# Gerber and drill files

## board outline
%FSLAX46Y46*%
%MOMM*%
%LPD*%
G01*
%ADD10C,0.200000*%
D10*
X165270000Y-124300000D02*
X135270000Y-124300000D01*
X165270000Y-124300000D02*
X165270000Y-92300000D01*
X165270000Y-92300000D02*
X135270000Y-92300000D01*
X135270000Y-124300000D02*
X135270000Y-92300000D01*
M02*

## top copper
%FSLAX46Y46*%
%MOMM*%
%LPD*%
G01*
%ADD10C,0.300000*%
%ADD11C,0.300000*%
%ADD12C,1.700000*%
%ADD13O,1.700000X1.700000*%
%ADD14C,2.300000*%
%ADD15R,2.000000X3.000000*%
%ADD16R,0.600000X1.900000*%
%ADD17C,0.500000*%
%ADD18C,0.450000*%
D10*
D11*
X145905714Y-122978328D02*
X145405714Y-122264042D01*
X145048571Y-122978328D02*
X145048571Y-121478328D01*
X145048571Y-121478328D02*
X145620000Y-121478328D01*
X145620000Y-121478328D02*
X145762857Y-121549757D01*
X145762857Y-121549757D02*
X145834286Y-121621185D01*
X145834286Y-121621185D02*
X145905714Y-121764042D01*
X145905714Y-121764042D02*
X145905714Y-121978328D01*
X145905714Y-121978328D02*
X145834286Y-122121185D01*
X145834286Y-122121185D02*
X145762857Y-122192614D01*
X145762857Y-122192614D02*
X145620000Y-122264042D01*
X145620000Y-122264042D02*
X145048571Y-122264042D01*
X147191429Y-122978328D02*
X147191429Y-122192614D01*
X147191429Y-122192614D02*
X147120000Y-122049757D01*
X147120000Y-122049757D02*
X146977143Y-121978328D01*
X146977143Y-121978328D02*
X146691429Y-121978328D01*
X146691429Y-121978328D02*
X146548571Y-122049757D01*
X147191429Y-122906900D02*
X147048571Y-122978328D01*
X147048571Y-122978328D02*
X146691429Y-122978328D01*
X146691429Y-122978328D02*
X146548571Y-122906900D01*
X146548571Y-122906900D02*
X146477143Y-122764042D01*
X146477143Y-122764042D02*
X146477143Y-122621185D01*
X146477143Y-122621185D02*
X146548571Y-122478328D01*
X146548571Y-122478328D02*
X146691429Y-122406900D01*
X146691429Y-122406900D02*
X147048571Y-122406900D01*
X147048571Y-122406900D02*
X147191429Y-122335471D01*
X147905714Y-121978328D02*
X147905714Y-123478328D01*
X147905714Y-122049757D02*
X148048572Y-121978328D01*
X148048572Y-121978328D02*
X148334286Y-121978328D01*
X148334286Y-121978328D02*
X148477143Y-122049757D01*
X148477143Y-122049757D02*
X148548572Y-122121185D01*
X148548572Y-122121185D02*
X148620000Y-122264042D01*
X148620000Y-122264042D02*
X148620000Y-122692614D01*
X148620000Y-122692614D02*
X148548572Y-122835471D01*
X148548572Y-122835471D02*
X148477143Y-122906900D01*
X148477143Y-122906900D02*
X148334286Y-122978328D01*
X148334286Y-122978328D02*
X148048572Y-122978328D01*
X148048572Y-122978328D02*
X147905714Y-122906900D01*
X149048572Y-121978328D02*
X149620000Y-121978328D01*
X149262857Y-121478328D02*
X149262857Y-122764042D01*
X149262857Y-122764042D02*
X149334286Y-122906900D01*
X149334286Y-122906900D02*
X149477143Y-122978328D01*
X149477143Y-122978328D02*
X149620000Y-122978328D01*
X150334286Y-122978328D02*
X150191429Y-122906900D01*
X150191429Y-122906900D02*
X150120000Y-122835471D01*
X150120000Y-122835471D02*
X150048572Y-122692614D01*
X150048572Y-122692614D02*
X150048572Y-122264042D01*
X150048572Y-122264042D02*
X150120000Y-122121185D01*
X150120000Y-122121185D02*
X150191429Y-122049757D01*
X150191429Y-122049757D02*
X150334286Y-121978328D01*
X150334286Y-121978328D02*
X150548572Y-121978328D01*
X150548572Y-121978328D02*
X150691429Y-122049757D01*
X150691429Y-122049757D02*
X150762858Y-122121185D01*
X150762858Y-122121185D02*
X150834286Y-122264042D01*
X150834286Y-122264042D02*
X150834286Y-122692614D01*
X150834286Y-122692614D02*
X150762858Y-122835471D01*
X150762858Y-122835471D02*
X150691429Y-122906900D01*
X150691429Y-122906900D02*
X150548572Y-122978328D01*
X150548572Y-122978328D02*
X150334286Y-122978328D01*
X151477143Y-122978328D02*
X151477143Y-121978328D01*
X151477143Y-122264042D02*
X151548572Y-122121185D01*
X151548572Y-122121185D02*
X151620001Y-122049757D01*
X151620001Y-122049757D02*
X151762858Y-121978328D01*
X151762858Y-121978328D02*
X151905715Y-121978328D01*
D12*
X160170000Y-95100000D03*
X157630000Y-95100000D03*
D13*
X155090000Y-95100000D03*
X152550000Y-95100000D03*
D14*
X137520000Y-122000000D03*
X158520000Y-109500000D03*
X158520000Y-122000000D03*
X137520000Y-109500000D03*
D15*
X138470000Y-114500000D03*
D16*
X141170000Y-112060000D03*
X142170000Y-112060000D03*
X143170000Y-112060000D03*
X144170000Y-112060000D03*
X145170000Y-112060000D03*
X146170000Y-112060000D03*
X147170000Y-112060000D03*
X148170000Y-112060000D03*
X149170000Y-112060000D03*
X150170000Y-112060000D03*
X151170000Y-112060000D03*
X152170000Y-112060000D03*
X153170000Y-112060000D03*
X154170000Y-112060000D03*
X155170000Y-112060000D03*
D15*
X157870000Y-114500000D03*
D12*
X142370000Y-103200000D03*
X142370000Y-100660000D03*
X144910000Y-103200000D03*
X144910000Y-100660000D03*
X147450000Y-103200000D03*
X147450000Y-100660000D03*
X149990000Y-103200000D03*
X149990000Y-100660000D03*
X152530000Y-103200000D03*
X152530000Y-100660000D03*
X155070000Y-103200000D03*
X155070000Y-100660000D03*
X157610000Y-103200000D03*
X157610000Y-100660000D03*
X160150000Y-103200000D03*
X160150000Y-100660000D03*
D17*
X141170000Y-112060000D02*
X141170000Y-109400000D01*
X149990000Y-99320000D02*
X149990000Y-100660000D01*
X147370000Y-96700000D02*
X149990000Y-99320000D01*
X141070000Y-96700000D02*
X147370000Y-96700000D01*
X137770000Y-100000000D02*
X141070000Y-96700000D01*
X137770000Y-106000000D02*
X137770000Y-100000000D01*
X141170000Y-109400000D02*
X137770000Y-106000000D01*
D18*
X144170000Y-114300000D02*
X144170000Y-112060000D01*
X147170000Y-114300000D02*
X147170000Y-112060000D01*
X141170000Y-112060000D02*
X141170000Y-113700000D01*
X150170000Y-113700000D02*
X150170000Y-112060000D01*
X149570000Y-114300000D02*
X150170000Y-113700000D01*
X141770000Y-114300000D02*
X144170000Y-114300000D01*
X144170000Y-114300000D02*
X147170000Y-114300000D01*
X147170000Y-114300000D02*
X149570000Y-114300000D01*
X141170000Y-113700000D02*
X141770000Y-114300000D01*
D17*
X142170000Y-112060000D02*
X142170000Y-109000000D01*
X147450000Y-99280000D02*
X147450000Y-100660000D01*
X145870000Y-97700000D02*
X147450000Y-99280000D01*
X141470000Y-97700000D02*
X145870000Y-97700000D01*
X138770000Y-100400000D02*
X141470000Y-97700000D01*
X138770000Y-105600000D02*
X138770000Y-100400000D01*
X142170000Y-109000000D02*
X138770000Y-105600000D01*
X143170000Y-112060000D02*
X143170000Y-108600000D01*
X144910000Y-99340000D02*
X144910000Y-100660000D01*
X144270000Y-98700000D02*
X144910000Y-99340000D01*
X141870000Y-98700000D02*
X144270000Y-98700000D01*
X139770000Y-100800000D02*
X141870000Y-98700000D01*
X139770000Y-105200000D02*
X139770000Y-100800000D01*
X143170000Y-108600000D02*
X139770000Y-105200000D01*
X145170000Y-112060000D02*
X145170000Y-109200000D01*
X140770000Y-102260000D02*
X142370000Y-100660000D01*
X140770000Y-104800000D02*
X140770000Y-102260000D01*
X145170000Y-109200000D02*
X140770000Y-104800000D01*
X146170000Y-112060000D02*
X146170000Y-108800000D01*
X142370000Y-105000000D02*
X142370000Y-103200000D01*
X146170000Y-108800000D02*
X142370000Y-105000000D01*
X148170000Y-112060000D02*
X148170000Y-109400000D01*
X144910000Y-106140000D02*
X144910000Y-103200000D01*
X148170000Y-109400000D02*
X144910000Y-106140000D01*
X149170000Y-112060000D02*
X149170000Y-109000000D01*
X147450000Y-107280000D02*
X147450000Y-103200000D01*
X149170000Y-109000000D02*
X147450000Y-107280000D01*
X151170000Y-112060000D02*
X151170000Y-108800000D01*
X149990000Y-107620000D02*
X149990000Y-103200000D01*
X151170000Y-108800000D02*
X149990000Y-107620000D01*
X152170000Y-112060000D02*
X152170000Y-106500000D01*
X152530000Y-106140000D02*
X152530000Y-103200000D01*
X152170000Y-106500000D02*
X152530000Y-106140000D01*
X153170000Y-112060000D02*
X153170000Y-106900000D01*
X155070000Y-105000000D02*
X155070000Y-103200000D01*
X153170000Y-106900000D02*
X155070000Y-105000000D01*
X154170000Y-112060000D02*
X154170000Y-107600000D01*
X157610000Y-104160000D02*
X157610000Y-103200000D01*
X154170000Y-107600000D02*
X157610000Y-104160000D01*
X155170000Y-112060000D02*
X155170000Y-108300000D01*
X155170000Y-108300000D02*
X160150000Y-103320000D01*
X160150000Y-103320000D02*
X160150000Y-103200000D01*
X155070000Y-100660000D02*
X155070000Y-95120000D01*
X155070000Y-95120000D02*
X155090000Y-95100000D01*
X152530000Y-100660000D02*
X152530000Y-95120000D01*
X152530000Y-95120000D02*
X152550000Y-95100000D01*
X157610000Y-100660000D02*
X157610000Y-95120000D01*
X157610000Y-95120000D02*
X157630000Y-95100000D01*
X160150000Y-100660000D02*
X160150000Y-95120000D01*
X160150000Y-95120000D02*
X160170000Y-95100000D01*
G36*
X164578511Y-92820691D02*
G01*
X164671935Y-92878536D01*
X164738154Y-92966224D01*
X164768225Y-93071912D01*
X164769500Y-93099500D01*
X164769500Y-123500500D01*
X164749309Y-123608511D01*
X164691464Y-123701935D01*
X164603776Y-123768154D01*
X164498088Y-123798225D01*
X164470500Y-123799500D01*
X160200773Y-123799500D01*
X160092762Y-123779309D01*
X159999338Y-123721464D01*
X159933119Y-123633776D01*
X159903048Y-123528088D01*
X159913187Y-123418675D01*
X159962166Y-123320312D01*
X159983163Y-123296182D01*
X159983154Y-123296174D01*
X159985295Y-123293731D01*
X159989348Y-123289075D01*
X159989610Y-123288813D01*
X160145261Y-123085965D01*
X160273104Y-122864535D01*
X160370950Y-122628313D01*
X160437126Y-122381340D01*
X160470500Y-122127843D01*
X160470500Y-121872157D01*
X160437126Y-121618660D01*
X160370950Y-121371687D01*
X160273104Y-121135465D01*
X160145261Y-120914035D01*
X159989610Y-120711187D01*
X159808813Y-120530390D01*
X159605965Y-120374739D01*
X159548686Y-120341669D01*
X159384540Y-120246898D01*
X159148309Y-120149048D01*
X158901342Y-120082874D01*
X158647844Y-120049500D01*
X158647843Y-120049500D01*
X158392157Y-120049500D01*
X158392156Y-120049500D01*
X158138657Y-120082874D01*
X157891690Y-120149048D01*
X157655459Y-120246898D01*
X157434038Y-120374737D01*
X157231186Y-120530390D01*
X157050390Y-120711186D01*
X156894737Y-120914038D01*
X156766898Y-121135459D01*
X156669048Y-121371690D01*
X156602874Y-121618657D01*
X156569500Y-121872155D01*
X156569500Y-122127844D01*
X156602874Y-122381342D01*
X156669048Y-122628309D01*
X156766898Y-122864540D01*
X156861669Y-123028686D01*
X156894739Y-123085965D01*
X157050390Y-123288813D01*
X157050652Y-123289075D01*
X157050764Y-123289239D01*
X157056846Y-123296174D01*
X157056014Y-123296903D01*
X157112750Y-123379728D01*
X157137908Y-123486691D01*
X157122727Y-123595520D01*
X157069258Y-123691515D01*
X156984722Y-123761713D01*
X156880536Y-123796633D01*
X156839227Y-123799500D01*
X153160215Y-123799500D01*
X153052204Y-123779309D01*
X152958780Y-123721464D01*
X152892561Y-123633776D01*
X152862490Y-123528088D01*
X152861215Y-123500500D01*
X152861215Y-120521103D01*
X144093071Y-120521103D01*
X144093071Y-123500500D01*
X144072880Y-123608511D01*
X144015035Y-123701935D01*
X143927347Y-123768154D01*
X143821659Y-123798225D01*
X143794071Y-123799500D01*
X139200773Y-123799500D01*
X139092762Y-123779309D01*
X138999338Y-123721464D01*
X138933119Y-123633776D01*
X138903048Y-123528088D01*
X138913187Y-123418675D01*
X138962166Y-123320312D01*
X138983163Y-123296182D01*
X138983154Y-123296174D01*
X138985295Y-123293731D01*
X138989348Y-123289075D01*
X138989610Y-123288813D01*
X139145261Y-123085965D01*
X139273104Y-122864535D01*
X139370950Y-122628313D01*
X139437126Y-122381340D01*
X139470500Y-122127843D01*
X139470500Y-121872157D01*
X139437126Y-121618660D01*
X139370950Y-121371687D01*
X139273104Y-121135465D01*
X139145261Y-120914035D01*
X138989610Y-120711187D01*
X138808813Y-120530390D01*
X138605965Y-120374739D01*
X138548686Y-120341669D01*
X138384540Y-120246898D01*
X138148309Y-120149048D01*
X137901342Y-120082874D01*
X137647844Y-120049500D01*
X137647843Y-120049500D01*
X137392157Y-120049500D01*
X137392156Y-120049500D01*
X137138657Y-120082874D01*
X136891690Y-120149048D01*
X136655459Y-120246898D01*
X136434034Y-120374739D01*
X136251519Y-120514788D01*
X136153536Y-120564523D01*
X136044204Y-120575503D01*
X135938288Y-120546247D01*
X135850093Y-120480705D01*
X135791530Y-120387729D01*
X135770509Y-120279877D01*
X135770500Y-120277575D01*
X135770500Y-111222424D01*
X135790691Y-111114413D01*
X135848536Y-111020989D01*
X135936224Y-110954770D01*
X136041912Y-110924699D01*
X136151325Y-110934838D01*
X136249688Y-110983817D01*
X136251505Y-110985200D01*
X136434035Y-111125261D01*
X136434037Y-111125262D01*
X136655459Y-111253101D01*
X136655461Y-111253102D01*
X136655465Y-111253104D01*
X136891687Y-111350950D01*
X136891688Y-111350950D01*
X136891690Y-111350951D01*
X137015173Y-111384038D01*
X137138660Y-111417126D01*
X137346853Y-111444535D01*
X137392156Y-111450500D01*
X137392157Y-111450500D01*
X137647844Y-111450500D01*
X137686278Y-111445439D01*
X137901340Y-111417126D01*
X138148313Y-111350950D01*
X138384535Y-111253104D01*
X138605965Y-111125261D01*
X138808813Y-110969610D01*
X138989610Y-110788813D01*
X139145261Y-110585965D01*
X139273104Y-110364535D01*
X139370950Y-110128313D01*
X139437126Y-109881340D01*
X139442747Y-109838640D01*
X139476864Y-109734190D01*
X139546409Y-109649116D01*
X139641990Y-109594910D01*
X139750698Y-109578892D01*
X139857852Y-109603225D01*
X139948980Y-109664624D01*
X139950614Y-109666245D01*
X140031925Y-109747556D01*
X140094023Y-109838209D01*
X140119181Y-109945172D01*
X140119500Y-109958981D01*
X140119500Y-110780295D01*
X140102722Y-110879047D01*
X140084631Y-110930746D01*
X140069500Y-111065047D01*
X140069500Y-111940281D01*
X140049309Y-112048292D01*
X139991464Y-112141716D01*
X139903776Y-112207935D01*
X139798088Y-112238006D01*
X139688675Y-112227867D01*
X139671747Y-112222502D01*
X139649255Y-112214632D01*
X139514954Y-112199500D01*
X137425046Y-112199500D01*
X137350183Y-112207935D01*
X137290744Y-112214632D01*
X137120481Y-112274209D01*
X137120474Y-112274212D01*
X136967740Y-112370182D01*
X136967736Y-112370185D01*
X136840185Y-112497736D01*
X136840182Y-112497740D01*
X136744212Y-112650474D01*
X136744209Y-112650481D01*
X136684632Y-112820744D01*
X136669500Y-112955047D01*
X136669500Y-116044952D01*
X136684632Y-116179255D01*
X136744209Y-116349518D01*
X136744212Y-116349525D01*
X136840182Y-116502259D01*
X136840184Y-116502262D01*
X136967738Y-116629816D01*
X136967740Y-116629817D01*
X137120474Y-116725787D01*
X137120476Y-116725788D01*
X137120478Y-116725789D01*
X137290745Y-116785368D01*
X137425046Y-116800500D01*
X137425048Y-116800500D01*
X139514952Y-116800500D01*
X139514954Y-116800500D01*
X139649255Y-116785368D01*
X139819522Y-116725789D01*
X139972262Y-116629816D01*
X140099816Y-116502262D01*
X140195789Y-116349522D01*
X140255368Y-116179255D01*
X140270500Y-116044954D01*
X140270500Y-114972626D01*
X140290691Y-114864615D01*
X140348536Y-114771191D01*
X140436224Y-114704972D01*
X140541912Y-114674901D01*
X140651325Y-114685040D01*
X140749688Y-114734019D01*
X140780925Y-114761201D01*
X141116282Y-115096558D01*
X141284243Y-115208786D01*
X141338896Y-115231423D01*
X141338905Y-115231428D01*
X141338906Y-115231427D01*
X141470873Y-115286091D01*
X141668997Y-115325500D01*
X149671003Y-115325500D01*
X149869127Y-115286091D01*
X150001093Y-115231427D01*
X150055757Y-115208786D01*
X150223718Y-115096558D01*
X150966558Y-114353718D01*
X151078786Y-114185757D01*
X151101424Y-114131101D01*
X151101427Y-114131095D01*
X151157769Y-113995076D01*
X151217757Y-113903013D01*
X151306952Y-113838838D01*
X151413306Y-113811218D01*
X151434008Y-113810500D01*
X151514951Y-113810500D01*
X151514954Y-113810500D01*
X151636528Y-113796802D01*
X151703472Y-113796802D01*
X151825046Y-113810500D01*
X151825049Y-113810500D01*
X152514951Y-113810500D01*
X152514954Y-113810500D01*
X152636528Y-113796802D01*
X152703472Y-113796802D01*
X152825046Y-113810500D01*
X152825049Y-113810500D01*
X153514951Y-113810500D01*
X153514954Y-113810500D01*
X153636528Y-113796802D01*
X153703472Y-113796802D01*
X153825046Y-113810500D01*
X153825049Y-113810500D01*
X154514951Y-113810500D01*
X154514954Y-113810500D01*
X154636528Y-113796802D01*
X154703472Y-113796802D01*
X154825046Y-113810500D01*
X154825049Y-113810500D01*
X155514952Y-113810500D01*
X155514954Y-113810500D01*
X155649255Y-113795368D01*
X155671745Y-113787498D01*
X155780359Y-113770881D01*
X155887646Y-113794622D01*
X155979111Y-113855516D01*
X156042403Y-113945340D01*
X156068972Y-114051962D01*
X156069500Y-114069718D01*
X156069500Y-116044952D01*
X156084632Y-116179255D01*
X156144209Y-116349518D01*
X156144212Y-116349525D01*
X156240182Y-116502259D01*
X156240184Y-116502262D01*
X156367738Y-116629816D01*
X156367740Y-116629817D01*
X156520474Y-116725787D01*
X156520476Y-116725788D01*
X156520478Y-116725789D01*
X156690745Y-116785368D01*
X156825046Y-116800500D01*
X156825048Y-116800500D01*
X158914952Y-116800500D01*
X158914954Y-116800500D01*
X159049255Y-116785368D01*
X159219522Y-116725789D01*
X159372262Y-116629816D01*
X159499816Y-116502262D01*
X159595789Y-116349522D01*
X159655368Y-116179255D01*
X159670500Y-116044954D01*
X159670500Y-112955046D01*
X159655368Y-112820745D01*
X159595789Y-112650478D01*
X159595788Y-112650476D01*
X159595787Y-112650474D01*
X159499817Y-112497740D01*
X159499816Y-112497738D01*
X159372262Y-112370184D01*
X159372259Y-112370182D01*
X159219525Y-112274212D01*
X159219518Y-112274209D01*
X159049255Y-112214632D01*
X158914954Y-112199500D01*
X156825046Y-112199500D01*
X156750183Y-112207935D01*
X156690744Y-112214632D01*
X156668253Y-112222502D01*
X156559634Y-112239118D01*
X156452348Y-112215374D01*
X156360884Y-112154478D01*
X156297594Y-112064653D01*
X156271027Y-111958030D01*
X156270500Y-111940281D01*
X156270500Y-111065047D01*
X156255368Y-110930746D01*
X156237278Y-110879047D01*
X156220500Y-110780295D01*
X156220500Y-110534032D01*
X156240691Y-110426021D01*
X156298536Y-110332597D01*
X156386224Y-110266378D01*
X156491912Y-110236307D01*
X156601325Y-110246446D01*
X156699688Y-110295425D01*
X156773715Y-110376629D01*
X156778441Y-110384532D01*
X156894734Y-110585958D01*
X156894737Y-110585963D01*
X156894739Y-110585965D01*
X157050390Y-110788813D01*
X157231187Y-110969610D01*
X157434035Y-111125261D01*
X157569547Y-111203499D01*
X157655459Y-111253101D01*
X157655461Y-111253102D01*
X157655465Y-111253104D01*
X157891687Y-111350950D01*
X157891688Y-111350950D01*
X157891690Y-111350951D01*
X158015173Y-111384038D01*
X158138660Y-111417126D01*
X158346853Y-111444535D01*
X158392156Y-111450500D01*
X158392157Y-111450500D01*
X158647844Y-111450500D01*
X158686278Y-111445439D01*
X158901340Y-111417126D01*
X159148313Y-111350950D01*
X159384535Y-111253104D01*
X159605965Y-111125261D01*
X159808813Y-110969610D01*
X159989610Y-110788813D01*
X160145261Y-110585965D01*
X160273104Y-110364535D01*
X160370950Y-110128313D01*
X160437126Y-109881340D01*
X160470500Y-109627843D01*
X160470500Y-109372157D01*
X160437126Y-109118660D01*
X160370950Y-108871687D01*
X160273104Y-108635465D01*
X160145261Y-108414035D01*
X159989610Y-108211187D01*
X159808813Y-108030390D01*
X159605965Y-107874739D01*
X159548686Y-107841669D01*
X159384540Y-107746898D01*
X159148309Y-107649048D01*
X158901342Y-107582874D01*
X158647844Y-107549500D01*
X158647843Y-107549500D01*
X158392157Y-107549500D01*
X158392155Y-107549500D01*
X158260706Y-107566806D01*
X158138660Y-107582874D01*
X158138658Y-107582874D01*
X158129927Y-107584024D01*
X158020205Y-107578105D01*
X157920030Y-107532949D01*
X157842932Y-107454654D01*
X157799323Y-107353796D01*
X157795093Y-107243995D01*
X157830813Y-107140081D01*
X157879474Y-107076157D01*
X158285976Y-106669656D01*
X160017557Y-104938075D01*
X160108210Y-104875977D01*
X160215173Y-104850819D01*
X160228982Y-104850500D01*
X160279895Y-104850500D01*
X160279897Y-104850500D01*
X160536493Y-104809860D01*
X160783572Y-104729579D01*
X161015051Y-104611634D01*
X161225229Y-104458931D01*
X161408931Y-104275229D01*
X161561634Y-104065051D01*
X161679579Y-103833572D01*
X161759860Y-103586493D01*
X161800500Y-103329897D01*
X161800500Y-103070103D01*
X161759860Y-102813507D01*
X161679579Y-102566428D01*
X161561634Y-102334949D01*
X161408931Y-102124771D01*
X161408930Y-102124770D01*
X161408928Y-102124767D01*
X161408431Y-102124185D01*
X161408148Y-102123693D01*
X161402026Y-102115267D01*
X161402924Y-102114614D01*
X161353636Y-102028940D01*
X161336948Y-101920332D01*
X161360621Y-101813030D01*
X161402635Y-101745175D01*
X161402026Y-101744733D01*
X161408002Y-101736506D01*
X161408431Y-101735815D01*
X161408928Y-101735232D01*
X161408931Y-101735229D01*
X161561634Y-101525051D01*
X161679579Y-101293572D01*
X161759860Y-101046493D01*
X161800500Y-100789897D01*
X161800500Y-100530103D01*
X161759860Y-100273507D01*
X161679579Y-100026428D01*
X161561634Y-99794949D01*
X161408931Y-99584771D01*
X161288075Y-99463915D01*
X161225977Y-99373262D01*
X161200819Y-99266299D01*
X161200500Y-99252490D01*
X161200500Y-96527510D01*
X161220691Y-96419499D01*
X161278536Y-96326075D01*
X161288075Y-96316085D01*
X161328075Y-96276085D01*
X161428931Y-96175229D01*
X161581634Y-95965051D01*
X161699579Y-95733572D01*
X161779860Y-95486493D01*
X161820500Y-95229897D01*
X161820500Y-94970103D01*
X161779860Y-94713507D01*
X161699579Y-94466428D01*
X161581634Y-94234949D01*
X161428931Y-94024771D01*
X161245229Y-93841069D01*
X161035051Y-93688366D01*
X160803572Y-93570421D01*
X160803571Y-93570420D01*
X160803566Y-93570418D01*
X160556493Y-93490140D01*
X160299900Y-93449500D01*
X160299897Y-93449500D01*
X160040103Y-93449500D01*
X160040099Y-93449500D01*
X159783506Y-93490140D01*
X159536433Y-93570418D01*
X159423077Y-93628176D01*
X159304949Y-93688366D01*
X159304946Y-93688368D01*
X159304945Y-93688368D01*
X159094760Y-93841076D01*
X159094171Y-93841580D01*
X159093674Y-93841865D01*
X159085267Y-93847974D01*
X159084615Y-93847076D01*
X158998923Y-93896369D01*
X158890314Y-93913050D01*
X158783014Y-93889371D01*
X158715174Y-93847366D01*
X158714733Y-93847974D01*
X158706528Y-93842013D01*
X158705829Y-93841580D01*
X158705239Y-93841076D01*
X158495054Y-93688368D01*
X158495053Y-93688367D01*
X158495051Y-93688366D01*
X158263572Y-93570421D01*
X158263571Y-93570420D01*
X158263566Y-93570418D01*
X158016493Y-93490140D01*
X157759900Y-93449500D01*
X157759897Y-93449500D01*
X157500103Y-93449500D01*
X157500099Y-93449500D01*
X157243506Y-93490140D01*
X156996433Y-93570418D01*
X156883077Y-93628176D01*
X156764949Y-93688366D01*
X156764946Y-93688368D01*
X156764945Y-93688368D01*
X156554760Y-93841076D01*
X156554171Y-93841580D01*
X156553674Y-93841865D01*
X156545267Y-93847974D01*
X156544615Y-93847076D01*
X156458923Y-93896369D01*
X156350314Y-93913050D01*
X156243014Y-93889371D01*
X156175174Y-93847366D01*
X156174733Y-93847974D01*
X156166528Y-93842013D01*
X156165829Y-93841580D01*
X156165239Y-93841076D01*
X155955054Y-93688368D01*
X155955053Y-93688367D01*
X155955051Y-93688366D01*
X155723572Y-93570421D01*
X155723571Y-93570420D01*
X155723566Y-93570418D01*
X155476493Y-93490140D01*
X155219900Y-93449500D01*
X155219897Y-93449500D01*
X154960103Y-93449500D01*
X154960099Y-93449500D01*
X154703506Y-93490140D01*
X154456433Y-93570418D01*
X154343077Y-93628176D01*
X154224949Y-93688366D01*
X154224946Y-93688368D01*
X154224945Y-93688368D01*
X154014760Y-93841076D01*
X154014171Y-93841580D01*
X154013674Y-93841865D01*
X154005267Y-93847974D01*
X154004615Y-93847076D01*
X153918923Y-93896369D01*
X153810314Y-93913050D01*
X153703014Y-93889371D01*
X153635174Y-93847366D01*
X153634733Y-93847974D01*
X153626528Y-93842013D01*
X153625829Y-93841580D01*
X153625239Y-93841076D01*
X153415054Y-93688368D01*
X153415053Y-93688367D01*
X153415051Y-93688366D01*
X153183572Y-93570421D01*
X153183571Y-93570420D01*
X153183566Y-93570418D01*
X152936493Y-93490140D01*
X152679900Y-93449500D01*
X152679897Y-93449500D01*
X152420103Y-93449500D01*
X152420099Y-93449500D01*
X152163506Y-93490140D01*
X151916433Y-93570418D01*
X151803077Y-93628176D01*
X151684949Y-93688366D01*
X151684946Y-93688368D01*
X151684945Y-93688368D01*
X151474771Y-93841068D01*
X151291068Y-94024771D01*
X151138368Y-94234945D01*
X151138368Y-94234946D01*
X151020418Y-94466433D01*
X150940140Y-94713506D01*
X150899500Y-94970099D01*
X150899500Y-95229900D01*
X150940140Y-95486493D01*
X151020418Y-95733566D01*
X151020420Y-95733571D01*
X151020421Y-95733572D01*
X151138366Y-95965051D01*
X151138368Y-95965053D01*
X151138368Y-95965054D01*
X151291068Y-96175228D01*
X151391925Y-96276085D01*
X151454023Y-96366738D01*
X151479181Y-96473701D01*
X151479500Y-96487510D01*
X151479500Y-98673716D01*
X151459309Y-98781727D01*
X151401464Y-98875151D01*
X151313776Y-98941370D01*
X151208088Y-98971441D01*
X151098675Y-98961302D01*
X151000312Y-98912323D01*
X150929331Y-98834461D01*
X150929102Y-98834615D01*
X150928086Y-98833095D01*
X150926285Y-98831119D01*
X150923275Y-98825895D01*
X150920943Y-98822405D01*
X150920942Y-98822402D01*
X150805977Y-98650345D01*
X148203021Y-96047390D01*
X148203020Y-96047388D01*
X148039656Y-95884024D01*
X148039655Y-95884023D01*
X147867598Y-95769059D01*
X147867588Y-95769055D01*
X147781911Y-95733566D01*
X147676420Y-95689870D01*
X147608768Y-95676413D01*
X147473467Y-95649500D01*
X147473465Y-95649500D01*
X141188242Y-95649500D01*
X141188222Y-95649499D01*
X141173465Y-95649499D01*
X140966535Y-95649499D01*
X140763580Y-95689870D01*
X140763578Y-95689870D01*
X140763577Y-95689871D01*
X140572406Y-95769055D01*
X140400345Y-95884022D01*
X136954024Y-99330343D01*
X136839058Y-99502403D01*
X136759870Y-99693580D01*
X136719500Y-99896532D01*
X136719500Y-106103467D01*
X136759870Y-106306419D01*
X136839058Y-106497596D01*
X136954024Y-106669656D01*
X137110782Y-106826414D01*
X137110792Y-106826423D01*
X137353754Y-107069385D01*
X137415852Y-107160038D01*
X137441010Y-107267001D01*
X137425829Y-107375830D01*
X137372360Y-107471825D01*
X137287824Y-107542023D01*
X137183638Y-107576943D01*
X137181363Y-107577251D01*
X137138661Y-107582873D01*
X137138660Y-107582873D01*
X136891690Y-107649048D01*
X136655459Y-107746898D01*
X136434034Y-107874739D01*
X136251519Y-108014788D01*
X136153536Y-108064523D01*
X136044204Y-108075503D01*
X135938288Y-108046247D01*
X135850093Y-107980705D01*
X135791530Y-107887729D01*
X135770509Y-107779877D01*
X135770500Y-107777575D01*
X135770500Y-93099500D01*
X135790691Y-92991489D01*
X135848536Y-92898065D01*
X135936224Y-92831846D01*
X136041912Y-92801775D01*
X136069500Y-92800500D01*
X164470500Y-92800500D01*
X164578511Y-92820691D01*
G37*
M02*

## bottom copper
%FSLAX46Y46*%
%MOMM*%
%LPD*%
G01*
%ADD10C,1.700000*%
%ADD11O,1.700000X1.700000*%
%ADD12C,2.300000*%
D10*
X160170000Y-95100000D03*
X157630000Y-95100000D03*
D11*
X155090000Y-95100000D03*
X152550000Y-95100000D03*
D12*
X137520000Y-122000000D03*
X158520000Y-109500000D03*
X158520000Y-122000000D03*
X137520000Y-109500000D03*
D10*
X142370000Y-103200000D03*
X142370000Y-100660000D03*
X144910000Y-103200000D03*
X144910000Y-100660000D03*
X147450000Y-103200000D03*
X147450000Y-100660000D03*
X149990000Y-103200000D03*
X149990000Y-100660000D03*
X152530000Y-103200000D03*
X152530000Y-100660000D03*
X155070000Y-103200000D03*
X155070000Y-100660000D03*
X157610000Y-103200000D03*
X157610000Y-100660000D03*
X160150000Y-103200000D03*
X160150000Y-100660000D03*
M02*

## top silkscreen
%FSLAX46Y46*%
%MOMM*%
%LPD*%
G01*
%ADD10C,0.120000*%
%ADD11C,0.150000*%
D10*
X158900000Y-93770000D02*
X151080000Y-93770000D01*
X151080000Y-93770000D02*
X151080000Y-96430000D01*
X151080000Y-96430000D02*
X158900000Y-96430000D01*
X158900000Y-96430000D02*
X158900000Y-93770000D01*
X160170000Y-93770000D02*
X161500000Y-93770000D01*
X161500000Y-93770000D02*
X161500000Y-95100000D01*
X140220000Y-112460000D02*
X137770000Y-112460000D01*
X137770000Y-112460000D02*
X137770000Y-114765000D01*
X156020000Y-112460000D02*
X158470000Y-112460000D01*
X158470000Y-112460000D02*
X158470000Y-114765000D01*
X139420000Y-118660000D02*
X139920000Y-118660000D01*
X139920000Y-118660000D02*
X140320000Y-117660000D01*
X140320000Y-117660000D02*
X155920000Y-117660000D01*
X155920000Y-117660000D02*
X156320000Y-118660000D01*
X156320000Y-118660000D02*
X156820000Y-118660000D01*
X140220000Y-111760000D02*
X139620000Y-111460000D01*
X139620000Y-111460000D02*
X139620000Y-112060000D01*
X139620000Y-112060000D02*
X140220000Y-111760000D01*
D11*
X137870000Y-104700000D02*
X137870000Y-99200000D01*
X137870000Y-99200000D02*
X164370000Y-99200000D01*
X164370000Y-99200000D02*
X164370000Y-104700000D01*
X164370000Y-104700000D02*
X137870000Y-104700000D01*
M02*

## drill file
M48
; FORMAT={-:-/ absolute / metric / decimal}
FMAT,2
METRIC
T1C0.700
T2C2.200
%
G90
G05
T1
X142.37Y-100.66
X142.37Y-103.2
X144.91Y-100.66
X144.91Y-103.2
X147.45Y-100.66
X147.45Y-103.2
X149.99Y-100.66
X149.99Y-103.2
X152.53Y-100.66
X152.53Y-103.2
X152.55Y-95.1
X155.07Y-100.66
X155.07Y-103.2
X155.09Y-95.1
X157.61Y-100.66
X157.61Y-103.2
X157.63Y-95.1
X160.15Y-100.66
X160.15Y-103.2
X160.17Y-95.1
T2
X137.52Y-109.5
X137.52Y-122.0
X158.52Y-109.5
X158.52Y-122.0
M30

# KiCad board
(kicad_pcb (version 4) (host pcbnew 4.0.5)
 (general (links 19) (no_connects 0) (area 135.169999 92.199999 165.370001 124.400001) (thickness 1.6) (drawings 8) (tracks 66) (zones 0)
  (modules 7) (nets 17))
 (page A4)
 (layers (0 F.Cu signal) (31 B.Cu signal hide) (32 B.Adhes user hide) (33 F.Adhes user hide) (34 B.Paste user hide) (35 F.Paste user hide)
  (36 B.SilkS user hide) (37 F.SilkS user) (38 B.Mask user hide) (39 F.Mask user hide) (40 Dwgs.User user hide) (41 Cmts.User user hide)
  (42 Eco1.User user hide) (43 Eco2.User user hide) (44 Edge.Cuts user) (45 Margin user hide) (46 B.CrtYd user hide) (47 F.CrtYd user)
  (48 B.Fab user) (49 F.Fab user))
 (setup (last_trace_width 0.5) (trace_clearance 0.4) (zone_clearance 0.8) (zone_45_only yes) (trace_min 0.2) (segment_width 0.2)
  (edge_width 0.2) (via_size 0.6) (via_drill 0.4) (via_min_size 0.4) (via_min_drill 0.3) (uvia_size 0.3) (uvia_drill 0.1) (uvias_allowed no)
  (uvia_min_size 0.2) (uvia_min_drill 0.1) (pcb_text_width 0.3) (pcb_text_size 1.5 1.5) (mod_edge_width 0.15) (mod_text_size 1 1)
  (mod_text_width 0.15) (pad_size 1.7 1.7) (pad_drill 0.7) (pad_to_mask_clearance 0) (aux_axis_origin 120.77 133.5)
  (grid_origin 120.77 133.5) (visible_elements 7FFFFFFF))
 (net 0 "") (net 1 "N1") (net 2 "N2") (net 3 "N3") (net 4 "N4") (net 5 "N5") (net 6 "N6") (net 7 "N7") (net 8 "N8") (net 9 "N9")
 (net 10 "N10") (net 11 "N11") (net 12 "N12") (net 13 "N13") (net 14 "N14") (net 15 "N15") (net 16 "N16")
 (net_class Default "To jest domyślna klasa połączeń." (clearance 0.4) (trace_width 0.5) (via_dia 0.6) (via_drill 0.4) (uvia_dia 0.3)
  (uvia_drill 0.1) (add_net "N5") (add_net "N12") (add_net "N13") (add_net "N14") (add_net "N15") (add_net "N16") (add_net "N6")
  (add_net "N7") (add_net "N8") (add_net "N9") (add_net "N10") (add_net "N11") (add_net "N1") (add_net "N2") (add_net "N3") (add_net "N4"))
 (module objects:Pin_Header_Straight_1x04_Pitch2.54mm (layer F.Cu) (at 160.17 95.1 270)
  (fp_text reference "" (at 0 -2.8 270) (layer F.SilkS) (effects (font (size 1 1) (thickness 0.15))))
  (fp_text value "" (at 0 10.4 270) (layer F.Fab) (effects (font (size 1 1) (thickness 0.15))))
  (fp_line (start -1.33 1.27) (end -1.33 9.09) (layer F.SilkS) (width 0.12))
  (fp_line (start -1.33 9.09) (end 1.33 9.09) (layer F.SilkS) (width 0.12))
  (fp_line (start 1.33 9.09) (end 1.33 1.27) (layer F.SilkS) (width 0.12))
  (fp_line (start 1.33 1.27) (end -1.33 1.27) (layer F.SilkS) (width 0.12))
  (fp_line (start -1.33 0) (end -1.33 -1.33) (layer F.SilkS) (width 0.12))
  (fp_line (start -1.33 -1.33) (end 0 -1.33) (layer F.SilkS) (width 0.12))
  (pad 1 thru_hole circle (at 0 0 270) (size 1.7 1.7) (drill 0.7) (layers *.Cu *.Mask) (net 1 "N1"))
  (pad 2 thru_hole circle (at 0 2.54 270) (size 1.7 1.7) (drill 0.7) (layers *.Cu *.Mask) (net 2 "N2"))
  (pad 3 thru_hole oval (at 0 5.08 270) (size 1.7 1.7) (drill 0.7) (layers *.Cu *.Mask) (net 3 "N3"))
  (pad 4 thru_hole oval (at 0 7.62 270) (size 1.7 1.7) (drill 0.7) (layers *.Cu *.Mask) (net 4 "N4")))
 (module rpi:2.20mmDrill (layer F.Cu) (at 137.52 122)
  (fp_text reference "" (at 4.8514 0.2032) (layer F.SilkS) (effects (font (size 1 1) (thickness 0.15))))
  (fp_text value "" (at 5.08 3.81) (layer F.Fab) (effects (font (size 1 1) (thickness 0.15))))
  (pad "" thru_hole circle (at 0 0) (size 2.3 2.3) (drill 2.2) (layers *.Cu *.Mask)))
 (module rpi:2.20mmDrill (layer F.Cu) (at 158.52 109.5)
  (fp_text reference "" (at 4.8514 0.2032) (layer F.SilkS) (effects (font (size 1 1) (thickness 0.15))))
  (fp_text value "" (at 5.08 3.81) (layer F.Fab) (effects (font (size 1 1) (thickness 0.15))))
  (pad "" thru_hole circle (at 0 0) (size 2.3 2.3) (drill 2.2) (layers *.Cu *.Mask)))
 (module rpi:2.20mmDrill (layer F.Cu) (at 158.52 122)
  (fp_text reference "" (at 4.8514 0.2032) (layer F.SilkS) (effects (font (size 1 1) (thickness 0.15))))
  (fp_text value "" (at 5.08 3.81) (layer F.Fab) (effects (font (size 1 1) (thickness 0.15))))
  (pad "" thru_hole circle (at 0 0) (size 2.3 2.3) (drill 2.2) (layers *.Cu *.Mask)))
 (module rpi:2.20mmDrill (layer F.Cu) (at 137.52 109.5)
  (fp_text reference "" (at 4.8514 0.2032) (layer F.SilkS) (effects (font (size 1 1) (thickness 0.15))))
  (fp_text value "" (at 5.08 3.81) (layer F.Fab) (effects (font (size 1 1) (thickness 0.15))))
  (pad "" thru_hole circle (at 0 0) (size 2.3 2.3) (drill 2.2) (layers *.Cu *.Mask)))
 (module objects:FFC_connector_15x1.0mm (layer F.Cu) (at 148.07 114.5)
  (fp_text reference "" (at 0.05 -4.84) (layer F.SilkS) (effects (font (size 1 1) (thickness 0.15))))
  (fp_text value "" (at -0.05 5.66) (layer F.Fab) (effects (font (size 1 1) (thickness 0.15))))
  (fp_line (start -7.85 -2.04) (end -10.3 -2.04) (layer F.SilkS) (width 0.12))
  (fp_line (start -10.3 -2.04) (end -10.3 0.265) (layer F.SilkS) (width 0.12))
  (fp_line (start 7.95 -2.04) (end 10.4 -2.04) (layer F.SilkS) (width 0.12))
  (fp_line (start 10.4 -2.04) (end 10.4 0.265) (layer F.SilkS) (width 0.12))
  (fp_line (start -8.65 4.16) (end -8.15 4.16) (layer F.SilkS) (width 0.12))
  (fp_line (start -8.15 4.16) (end -7.75 3.16) (layer F.SilkS) (width 0.12))
  (fp_line (start -7.75 3.16) (end 7.85 3.16) (layer F.SilkS) (width 0.12))
  (fp_line (start 7.85 3.16) (end 8.25 4.16) (layer F.SilkS) (width 0.12))
  (fp_line (start 8.25 4.16) (end 8.75 4.16) (layer F.SilkS) (width 0.12))
  (fp_line (start -7.85 -2.74) (end -8.45 -3.04) (layer F.SilkS) (width 0.12))
  (fp_line (start -8.45 -3.04) (end -8.45 -2.44) (layer F.SilkS) (width 0.12))
  (fp_line (start -8.45 -2.44) (end -7.85 -2.74) (layer F.SilkS) (width 0.12))
  (pad "" smd rect (at -9.6 0) (size 2 3) (layers F.Cu F.Paste F.Mask))
  (pad 1 smd rect (at -6.9 -2.44) (size 0.6 1.9) (layers F.Cu F.Paste F.Mask) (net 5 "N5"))
  (pad 2 smd rect (at -5.9 -2.44) (size 0.6 1.9) (layers F.Cu F.Paste F.Mask) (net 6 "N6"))
  (pad 3 smd rect (at -4.9 -2.44) (size 0.6 1.9) (layers F.Cu F.Paste F.Mask) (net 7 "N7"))
  (pad 4 smd rect (at -3.9 -2.44) (size 0.6 1.9) (layers F.Cu F.Paste F.Mask) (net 5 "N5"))
  (pad 5 smd rect (at -2.9 -2.44) (size 0.6 1.9) (layers F.Cu F.Paste F.Mask) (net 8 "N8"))
  (pad 6 smd rect (at -1.9 -2.44) (size 0.6 1.9) (layers F.Cu F.Paste F.Mask) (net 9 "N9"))
  (pad 7 smd rect (at -0.9 -2.44) (size 0.6 1.9) (layers F.Cu F.Paste F.Mask) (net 5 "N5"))
  (pad 8 smd rect (at 0.1 -2.44) (size 0.6 1.9) (layers F.Cu F.Paste F.Mask) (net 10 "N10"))
  (pad 9 smd rect (at 1.1 -2.44) (size 0.6 1.9) (layers F.Cu F.Paste F.Mask) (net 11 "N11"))
  (pad 10 smd rect (at 2.1 -2.44) (size 0.6 1.9) (layers F.Cu F.Paste F.Mask) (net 5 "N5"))
  (pad 11 smd rect (at 3.1 -2.44) (size 0.6 1.9) (layers F.Cu F.Paste F.Mask) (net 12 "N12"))
  (pad 12 smd rect (at 4.1 -2.44) (size 0.6 1.9) (layers F.Cu F.Paste F.Mask) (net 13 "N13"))
  (pad 13 smd rect (at 5.1 -2.44) (size 0.6 1.9) (layers F.Cu F.Paste F.Mask) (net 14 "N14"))
  (pad 14 smd rect (at 6.1 -2.44) (size 0.6 1.9) (layers F.Cu F.Paste F.Mask) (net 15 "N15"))
  (pad 15 smd rect (at 7.1 -2.44) (size 0.6 1.9) (layers F.Cu F.Paste F.Mask) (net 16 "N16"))
  (pad "" smd rect (at 9.8 0) (size 2 3) (layers F.Cu F.Paste F.Mask)))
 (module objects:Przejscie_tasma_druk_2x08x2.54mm (layer F.Cu) (at 142.37 103.2)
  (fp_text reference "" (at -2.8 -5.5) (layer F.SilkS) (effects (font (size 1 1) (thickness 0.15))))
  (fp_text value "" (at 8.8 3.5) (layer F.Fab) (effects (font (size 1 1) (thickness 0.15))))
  (fp_line (start -4.5 1.5) (end -4.5 -4) (layer F.SilkS) (width 0.15))
  (fp_line (start -4.5 -4) (end 22 -4) (layer F.SilkS) (width 0.15))
  (fp_line (start 22 -4) (end 22 1.5) (layer F.SilkS) (width 0.15))
  (fp_line (start 22 1.5) (end -4.5 1.5) (layer F.SilkS) (width 0.15))
  (pad 1 thru_hole circle (at 0 0) (size 1.7 1.7) (drill 0.7) (layers *.Cu *.Mask) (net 9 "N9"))
  (pad 2 thru_hole circle (at 0 -2.54) (size 1.7 1.7) (drill 0.7) (layers *.Cu *.Mask) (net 8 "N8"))
  (pad 3 thru_hole circle (at 2.54 0) (size 1.7 1.7) (drill 0.7) (layers *.Cu *.Mask) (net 10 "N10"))
  (pad 4 thru_hole circle (at 2.54 -2.54) (size 1.7 1.7) (drill 0.7) (layers *.Cu *.Mask) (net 7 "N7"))
  (pad 5 thru_hole circle (at 5.08 0) (size 1.7 1.7) (drill 0.7) (layers *.Cu *.Mask) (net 11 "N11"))
  (pad 6 thru_hole circle (at 5.08 -2.54) (size 1.7 1.7) (drill 0.7) (layers *.Cu *.Mask) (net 6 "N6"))
  (pad 7 thru_hole circle (at 7.62 0) (size 1.7 1.7) (drill 0.7) (layers *.Cu *.Mask) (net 12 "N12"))
  (pad 8 thru_hole circle (at 7.62 -2.54) (size 1.7 1.7) (drill 0.7) (layers *.Cu *.Mask) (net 5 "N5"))
  (pad 9 thru_hole circle (at 10.16 0) (size 1.7 1.7) (drill 0.7) (layers *.Cu *.Mask) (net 13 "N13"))
  (pad 10 thru_hole circle (at 10.16 -2.54) (size 1.7 1.7) (drill 0.7) (layers *.Cu *.Mask) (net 4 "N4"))
  (pad 11 thru_hole circle (at 12.7 0) (size 1.7 1.7) (drill 0.7) (layers *.Cu *.Mask) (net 14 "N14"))
  (pad 12 thru_hole circle (at 12.7 -2.54) (size 1.7 1.7) (drill 0.7) (layers *.Cu *.Mask) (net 3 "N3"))
  (pad 13 thru_hole circle (at 15.24 0) (size 1.7 1.7) (drill 0.7) (layers *.Cu *.Mask) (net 15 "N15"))
  (pad 14 thru_hole circle (at 15.24 -2.54) (size 1.7 1.7) (drill 0.7) (layers *.Cu *.Mask) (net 2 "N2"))
  (pad 15 thru_hole circle (at 17.78 0) (size 1.7 1.7) (drill 0.7) (layers *.Cu *.Mask) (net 16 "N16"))
  (pad 16 thru_hole circle (at 17.78 -2.54) (size 1.7 1.7) (drill 0.7) (layers *.Cu *.Mask) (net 1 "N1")))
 (gr_line (start 165.27 124.3) (end 135.27 124.3) (angle 90) (layer Edge.Cuts) (width 0.2))
 (gr_line (start 165.27 124.3) (end 165.27 92.3) (angle 90) (layer Edge.Cuts) (width 0.2))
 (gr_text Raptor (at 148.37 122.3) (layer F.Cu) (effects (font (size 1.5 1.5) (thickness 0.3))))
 (gr_line (start 165.27 92.3) (end 135.27 92.3) (angle 90) (layer Edge.Cuts) (width 0.2))
 (gr_line (start 135.27 124.3) (end 135.27 92.3) (angle 90) (layer Edge.Cuts) (width 0.2))
 (segment (start 141.17 112.06) (end 141.17 109.4) (width 0.5) (layer F.Cu) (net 5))
 (segment (start 149.99 99.32) (end 149.99 100.66) (width 0.5) (layer F.Cu) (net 5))
 (segment (start 147.37 96.7) (end 149.99 99.32) (width 0.5) (layer F.Cu) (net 5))
 (segment (start 141.07 96.7) (end 147.37 96.7) (width 0.5) (layer F.Cu) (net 5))
 (segment (start 137.77 100) (end 141.07 96.7) (width 0.5) (layer F.Cu) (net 5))
 (segment (start 137.77 106) (end 137.77 100) (width 0.5) (layer F.Cu) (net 5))
 (segment (start 141.17 109.4) (end 137.77 106) (width 0.5) (layer F.Cu) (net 5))
 (segment (start 144.17 114.3) (end 144.17 112.06) (width 0.45) (layer F.Cu) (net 5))
 (segment (start 147.17 114.3) (end 147.17 112.06) (width 0.45) (layer F.Cu) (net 5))
 (segment (start 141.17 112.06) (end 141.17 113.7) (width 0.45) (layer F.Cu) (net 5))
 (segment (start 150.17 113.7) (end 150.17 112.06) (width 0.45) (layer F.Cu) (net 5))
 (segment (start 149.57 114.3) (end 150.17 113.7) (width 0.45) (layer F.Cu) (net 5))
 (segment (start 141.77 114.3) (end 144.17 114.3) (width 0.45) (layer F.Cu) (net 5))
 (segment (start 144.17 114.3) (end 147.17 114.3) (width 0.45) (layer F.Cu) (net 5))
 (segment (start 147.17 114.3) (end 149.57 114.3) (width 0.45) (layer F.Cu) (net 5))
 (segment (start 141.17 113.7) (end 141.77 114.3) (width 0.45) (layer F.Cu) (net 5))
 (segment (start 142.17 112.06) (end 142.17 109) (width 0.5) (layer F.Cu) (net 6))
 (segment (start 147.45 99.28) (end 147.45 100.66) (width 0.5) (layer F.Cu) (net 6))
 (segment (start 145.87 97.7) (end 147.45 99.28) (width 0.5) (layer F.Cu) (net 6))
 (segment (start 141.47 97.7) (end 145.87 97.7) (width 0.5) (layer F.Cu) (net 6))
 (segment (start 138.77 100.4) (end 141.47 97.7) (width 0.5) (layer F.Cu) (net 6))
 (segment (start 138.77 105.6) (end 138.77 100.4) (width 0.5) (layer F.Cu) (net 6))
 (segment (start 142.17 109) (end 138.77 105.6) (width 0.5) (layer F.Cu) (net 6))
 (segment (start 143.17 112.06) (end 143.17 108.6) (width 0.5) (layer F.Cu) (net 7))
 (segment (start 144.91 99.34) (end 144.91 100.66) (width 0.5) (layer F.Cu) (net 7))
 (segment (start 144.27 98.7) (end 144.91 99.34) (width 0.5) (layer F.Cu) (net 7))
 (segment (start 141.87 98.7) (end 144.27 98.7) (width 0.5) (layer F.Cu) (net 7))
 (segment (start 139.77 100.8) (end 141.87 98.7) (width 0.5) (layer F.Cu) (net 7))
 (segment (start 139.77 105.2) (end 139.77 100.8) (width 0.5) (layer F.Cu) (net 7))
 (segment (start 143.17 108.6) (end 139.77 105.2) (width 0.5) (layer F.Cu) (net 7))
 (segment (start 145.17 112.06) (end 145.17 109.2) (width 0.5) (layer F.Cu) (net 8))
 (segment (start 140.77 102.26) (end 142.37 100.66) (width 0.5) (layer F.Cu) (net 8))
 (segment (start 140.77 104.8) (end 140.77 102.26) (width 0.5) (layer F.Cu) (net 8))
 (segment (start 145.17 109.2) (end 140.77 104.8) (width 0.5) (layer F.Cu) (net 8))
 (segment (start 146.17 112.06) (end 146.17 108.8) (width 0.5) (layer F.Cu) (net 9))
 (segment (start 142.37 105) (end 142.37 103.2) (width 0.5) (layer F.Cu) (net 9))
 (segment (start 146.17 108.8) (end 142.37 105) (width 0.5) (layer F.Cu) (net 9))
 (segment (start 148.17 112.06) (end 148.17 109.4) (width 0.5) (layer F.Cu) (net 10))
 (segment (start 144.91 106.14) (end 144.91 103.2) (width 0.5) (layer F.Cu) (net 10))
 (segment (start 148.17 109.4) (end 144.91 106.14) (width 0.5) (layer F.Cu) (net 10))
 (segment (start 149.17 112.06) (end 149.17 109) (width 0.5) (layer F.Cu) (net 11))
 (segment (start 147.45 107.28) (end 147.45 103.2) (width 0.5) (layer F.Cu) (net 11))
 (segment (start 149.17 109) (end 147.45 107.28) (width 0.5) (layer F.Cu) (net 11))
 (segment (start 151.17 112.06) (end 151.17 108.8) (width 0.5) (layer F.Cu) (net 12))
 (segment (start 149.99 107.62) (end 149.99 103.2) (width 0.5) (layer F.Cu) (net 12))
 (segment (start 151.17 108.8) (end 149.99 107.62) (width 0.5) (layer F.Cu) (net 12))
 (segment (start 152.17 112.06) (end 152.17 106.5) (width 0.5) (layer F.Cu) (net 13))
 (segment (start 152.53 106.14) (end 152.53 103.2) (width 0.5) (layer F.Cu) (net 13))
 (segment (start 152.17 106.5) (end 152.53 106.14) (width 0.5) (layer F.Cu) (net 13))
 (segment (start 153.17 112.06) (end 153.17 106.9) (width 0.5) (layer F.Cu) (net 14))
 (segment (start 155.07 105) (end 155.07 103.2) (width 0.5) (layer F.Cu) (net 14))
 (segment (start 153.17 106.9) (end 155.07 105) (width 0.5) (layer F.Cu) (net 14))
 (segment (start 154.17 112.06) (end 154.17 107.6) (width 0.5) (layer F.Cu) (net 15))
 (segment (start 157.61 104.16) (end 157.61 103.2) (width 0.5) (layer F.Cu) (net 15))
 (segment (start 154.17 107.6) (end 157.61 104.16) (width 0.5) (layer F.Cu) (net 15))
 (segment (start 155.17 112.06) (end 155.17 108.3) (width 0.5) (layer F.Cu) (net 16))
 (segment (start 155.17 108.3) (end 160.15 103.32) (width 0.5) (layer F.Cu) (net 16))
 (segment (start 160.15 103.32) (end 160.15 103.2) (width 0.5) (layer F.Cu) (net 16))
 (segment (start 155.07 100.66) (end 155.07 95.12) (width 0.5) (layer F.Cu) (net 3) (status C00000))
 (segment (start 155.07 95.12) (end 155.09 95.1) (width 0.5) (layer F.Cu) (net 3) (status C00000))
 (segment (start 152.53 100.66) (end 152.53 95.12) (width 0.5) (layer F.Cu) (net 4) (status C00000))
 (segment (start 152.53 95.12) (end 152.55 95.1) (width 0.5) (layer F.Cu) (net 4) (status C00000))
 (segment (start 157.61 100.66) (end 157.61 95.12) (width 0.5) (layer F.Cu) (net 2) (status C00000))
 (segment (start 157.61 95.12) (end 157.63 95.1) (width 0.5) (layer F.Cu) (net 2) (status C00000))
 (segment (start 160.15 100.66) (end 160.15 95.12) (width 0.5) (layer F.Cu) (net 1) (status C00000))
 (segment (start 160.15 95.12) (end 160.17 95.1) (width 0.5) (layer F.Cu) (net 1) (status C00000))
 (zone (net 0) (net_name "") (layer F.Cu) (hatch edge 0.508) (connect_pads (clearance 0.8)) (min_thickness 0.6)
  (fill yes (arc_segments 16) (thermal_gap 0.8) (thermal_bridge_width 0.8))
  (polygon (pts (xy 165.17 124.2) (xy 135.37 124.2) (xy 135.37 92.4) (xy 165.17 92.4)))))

